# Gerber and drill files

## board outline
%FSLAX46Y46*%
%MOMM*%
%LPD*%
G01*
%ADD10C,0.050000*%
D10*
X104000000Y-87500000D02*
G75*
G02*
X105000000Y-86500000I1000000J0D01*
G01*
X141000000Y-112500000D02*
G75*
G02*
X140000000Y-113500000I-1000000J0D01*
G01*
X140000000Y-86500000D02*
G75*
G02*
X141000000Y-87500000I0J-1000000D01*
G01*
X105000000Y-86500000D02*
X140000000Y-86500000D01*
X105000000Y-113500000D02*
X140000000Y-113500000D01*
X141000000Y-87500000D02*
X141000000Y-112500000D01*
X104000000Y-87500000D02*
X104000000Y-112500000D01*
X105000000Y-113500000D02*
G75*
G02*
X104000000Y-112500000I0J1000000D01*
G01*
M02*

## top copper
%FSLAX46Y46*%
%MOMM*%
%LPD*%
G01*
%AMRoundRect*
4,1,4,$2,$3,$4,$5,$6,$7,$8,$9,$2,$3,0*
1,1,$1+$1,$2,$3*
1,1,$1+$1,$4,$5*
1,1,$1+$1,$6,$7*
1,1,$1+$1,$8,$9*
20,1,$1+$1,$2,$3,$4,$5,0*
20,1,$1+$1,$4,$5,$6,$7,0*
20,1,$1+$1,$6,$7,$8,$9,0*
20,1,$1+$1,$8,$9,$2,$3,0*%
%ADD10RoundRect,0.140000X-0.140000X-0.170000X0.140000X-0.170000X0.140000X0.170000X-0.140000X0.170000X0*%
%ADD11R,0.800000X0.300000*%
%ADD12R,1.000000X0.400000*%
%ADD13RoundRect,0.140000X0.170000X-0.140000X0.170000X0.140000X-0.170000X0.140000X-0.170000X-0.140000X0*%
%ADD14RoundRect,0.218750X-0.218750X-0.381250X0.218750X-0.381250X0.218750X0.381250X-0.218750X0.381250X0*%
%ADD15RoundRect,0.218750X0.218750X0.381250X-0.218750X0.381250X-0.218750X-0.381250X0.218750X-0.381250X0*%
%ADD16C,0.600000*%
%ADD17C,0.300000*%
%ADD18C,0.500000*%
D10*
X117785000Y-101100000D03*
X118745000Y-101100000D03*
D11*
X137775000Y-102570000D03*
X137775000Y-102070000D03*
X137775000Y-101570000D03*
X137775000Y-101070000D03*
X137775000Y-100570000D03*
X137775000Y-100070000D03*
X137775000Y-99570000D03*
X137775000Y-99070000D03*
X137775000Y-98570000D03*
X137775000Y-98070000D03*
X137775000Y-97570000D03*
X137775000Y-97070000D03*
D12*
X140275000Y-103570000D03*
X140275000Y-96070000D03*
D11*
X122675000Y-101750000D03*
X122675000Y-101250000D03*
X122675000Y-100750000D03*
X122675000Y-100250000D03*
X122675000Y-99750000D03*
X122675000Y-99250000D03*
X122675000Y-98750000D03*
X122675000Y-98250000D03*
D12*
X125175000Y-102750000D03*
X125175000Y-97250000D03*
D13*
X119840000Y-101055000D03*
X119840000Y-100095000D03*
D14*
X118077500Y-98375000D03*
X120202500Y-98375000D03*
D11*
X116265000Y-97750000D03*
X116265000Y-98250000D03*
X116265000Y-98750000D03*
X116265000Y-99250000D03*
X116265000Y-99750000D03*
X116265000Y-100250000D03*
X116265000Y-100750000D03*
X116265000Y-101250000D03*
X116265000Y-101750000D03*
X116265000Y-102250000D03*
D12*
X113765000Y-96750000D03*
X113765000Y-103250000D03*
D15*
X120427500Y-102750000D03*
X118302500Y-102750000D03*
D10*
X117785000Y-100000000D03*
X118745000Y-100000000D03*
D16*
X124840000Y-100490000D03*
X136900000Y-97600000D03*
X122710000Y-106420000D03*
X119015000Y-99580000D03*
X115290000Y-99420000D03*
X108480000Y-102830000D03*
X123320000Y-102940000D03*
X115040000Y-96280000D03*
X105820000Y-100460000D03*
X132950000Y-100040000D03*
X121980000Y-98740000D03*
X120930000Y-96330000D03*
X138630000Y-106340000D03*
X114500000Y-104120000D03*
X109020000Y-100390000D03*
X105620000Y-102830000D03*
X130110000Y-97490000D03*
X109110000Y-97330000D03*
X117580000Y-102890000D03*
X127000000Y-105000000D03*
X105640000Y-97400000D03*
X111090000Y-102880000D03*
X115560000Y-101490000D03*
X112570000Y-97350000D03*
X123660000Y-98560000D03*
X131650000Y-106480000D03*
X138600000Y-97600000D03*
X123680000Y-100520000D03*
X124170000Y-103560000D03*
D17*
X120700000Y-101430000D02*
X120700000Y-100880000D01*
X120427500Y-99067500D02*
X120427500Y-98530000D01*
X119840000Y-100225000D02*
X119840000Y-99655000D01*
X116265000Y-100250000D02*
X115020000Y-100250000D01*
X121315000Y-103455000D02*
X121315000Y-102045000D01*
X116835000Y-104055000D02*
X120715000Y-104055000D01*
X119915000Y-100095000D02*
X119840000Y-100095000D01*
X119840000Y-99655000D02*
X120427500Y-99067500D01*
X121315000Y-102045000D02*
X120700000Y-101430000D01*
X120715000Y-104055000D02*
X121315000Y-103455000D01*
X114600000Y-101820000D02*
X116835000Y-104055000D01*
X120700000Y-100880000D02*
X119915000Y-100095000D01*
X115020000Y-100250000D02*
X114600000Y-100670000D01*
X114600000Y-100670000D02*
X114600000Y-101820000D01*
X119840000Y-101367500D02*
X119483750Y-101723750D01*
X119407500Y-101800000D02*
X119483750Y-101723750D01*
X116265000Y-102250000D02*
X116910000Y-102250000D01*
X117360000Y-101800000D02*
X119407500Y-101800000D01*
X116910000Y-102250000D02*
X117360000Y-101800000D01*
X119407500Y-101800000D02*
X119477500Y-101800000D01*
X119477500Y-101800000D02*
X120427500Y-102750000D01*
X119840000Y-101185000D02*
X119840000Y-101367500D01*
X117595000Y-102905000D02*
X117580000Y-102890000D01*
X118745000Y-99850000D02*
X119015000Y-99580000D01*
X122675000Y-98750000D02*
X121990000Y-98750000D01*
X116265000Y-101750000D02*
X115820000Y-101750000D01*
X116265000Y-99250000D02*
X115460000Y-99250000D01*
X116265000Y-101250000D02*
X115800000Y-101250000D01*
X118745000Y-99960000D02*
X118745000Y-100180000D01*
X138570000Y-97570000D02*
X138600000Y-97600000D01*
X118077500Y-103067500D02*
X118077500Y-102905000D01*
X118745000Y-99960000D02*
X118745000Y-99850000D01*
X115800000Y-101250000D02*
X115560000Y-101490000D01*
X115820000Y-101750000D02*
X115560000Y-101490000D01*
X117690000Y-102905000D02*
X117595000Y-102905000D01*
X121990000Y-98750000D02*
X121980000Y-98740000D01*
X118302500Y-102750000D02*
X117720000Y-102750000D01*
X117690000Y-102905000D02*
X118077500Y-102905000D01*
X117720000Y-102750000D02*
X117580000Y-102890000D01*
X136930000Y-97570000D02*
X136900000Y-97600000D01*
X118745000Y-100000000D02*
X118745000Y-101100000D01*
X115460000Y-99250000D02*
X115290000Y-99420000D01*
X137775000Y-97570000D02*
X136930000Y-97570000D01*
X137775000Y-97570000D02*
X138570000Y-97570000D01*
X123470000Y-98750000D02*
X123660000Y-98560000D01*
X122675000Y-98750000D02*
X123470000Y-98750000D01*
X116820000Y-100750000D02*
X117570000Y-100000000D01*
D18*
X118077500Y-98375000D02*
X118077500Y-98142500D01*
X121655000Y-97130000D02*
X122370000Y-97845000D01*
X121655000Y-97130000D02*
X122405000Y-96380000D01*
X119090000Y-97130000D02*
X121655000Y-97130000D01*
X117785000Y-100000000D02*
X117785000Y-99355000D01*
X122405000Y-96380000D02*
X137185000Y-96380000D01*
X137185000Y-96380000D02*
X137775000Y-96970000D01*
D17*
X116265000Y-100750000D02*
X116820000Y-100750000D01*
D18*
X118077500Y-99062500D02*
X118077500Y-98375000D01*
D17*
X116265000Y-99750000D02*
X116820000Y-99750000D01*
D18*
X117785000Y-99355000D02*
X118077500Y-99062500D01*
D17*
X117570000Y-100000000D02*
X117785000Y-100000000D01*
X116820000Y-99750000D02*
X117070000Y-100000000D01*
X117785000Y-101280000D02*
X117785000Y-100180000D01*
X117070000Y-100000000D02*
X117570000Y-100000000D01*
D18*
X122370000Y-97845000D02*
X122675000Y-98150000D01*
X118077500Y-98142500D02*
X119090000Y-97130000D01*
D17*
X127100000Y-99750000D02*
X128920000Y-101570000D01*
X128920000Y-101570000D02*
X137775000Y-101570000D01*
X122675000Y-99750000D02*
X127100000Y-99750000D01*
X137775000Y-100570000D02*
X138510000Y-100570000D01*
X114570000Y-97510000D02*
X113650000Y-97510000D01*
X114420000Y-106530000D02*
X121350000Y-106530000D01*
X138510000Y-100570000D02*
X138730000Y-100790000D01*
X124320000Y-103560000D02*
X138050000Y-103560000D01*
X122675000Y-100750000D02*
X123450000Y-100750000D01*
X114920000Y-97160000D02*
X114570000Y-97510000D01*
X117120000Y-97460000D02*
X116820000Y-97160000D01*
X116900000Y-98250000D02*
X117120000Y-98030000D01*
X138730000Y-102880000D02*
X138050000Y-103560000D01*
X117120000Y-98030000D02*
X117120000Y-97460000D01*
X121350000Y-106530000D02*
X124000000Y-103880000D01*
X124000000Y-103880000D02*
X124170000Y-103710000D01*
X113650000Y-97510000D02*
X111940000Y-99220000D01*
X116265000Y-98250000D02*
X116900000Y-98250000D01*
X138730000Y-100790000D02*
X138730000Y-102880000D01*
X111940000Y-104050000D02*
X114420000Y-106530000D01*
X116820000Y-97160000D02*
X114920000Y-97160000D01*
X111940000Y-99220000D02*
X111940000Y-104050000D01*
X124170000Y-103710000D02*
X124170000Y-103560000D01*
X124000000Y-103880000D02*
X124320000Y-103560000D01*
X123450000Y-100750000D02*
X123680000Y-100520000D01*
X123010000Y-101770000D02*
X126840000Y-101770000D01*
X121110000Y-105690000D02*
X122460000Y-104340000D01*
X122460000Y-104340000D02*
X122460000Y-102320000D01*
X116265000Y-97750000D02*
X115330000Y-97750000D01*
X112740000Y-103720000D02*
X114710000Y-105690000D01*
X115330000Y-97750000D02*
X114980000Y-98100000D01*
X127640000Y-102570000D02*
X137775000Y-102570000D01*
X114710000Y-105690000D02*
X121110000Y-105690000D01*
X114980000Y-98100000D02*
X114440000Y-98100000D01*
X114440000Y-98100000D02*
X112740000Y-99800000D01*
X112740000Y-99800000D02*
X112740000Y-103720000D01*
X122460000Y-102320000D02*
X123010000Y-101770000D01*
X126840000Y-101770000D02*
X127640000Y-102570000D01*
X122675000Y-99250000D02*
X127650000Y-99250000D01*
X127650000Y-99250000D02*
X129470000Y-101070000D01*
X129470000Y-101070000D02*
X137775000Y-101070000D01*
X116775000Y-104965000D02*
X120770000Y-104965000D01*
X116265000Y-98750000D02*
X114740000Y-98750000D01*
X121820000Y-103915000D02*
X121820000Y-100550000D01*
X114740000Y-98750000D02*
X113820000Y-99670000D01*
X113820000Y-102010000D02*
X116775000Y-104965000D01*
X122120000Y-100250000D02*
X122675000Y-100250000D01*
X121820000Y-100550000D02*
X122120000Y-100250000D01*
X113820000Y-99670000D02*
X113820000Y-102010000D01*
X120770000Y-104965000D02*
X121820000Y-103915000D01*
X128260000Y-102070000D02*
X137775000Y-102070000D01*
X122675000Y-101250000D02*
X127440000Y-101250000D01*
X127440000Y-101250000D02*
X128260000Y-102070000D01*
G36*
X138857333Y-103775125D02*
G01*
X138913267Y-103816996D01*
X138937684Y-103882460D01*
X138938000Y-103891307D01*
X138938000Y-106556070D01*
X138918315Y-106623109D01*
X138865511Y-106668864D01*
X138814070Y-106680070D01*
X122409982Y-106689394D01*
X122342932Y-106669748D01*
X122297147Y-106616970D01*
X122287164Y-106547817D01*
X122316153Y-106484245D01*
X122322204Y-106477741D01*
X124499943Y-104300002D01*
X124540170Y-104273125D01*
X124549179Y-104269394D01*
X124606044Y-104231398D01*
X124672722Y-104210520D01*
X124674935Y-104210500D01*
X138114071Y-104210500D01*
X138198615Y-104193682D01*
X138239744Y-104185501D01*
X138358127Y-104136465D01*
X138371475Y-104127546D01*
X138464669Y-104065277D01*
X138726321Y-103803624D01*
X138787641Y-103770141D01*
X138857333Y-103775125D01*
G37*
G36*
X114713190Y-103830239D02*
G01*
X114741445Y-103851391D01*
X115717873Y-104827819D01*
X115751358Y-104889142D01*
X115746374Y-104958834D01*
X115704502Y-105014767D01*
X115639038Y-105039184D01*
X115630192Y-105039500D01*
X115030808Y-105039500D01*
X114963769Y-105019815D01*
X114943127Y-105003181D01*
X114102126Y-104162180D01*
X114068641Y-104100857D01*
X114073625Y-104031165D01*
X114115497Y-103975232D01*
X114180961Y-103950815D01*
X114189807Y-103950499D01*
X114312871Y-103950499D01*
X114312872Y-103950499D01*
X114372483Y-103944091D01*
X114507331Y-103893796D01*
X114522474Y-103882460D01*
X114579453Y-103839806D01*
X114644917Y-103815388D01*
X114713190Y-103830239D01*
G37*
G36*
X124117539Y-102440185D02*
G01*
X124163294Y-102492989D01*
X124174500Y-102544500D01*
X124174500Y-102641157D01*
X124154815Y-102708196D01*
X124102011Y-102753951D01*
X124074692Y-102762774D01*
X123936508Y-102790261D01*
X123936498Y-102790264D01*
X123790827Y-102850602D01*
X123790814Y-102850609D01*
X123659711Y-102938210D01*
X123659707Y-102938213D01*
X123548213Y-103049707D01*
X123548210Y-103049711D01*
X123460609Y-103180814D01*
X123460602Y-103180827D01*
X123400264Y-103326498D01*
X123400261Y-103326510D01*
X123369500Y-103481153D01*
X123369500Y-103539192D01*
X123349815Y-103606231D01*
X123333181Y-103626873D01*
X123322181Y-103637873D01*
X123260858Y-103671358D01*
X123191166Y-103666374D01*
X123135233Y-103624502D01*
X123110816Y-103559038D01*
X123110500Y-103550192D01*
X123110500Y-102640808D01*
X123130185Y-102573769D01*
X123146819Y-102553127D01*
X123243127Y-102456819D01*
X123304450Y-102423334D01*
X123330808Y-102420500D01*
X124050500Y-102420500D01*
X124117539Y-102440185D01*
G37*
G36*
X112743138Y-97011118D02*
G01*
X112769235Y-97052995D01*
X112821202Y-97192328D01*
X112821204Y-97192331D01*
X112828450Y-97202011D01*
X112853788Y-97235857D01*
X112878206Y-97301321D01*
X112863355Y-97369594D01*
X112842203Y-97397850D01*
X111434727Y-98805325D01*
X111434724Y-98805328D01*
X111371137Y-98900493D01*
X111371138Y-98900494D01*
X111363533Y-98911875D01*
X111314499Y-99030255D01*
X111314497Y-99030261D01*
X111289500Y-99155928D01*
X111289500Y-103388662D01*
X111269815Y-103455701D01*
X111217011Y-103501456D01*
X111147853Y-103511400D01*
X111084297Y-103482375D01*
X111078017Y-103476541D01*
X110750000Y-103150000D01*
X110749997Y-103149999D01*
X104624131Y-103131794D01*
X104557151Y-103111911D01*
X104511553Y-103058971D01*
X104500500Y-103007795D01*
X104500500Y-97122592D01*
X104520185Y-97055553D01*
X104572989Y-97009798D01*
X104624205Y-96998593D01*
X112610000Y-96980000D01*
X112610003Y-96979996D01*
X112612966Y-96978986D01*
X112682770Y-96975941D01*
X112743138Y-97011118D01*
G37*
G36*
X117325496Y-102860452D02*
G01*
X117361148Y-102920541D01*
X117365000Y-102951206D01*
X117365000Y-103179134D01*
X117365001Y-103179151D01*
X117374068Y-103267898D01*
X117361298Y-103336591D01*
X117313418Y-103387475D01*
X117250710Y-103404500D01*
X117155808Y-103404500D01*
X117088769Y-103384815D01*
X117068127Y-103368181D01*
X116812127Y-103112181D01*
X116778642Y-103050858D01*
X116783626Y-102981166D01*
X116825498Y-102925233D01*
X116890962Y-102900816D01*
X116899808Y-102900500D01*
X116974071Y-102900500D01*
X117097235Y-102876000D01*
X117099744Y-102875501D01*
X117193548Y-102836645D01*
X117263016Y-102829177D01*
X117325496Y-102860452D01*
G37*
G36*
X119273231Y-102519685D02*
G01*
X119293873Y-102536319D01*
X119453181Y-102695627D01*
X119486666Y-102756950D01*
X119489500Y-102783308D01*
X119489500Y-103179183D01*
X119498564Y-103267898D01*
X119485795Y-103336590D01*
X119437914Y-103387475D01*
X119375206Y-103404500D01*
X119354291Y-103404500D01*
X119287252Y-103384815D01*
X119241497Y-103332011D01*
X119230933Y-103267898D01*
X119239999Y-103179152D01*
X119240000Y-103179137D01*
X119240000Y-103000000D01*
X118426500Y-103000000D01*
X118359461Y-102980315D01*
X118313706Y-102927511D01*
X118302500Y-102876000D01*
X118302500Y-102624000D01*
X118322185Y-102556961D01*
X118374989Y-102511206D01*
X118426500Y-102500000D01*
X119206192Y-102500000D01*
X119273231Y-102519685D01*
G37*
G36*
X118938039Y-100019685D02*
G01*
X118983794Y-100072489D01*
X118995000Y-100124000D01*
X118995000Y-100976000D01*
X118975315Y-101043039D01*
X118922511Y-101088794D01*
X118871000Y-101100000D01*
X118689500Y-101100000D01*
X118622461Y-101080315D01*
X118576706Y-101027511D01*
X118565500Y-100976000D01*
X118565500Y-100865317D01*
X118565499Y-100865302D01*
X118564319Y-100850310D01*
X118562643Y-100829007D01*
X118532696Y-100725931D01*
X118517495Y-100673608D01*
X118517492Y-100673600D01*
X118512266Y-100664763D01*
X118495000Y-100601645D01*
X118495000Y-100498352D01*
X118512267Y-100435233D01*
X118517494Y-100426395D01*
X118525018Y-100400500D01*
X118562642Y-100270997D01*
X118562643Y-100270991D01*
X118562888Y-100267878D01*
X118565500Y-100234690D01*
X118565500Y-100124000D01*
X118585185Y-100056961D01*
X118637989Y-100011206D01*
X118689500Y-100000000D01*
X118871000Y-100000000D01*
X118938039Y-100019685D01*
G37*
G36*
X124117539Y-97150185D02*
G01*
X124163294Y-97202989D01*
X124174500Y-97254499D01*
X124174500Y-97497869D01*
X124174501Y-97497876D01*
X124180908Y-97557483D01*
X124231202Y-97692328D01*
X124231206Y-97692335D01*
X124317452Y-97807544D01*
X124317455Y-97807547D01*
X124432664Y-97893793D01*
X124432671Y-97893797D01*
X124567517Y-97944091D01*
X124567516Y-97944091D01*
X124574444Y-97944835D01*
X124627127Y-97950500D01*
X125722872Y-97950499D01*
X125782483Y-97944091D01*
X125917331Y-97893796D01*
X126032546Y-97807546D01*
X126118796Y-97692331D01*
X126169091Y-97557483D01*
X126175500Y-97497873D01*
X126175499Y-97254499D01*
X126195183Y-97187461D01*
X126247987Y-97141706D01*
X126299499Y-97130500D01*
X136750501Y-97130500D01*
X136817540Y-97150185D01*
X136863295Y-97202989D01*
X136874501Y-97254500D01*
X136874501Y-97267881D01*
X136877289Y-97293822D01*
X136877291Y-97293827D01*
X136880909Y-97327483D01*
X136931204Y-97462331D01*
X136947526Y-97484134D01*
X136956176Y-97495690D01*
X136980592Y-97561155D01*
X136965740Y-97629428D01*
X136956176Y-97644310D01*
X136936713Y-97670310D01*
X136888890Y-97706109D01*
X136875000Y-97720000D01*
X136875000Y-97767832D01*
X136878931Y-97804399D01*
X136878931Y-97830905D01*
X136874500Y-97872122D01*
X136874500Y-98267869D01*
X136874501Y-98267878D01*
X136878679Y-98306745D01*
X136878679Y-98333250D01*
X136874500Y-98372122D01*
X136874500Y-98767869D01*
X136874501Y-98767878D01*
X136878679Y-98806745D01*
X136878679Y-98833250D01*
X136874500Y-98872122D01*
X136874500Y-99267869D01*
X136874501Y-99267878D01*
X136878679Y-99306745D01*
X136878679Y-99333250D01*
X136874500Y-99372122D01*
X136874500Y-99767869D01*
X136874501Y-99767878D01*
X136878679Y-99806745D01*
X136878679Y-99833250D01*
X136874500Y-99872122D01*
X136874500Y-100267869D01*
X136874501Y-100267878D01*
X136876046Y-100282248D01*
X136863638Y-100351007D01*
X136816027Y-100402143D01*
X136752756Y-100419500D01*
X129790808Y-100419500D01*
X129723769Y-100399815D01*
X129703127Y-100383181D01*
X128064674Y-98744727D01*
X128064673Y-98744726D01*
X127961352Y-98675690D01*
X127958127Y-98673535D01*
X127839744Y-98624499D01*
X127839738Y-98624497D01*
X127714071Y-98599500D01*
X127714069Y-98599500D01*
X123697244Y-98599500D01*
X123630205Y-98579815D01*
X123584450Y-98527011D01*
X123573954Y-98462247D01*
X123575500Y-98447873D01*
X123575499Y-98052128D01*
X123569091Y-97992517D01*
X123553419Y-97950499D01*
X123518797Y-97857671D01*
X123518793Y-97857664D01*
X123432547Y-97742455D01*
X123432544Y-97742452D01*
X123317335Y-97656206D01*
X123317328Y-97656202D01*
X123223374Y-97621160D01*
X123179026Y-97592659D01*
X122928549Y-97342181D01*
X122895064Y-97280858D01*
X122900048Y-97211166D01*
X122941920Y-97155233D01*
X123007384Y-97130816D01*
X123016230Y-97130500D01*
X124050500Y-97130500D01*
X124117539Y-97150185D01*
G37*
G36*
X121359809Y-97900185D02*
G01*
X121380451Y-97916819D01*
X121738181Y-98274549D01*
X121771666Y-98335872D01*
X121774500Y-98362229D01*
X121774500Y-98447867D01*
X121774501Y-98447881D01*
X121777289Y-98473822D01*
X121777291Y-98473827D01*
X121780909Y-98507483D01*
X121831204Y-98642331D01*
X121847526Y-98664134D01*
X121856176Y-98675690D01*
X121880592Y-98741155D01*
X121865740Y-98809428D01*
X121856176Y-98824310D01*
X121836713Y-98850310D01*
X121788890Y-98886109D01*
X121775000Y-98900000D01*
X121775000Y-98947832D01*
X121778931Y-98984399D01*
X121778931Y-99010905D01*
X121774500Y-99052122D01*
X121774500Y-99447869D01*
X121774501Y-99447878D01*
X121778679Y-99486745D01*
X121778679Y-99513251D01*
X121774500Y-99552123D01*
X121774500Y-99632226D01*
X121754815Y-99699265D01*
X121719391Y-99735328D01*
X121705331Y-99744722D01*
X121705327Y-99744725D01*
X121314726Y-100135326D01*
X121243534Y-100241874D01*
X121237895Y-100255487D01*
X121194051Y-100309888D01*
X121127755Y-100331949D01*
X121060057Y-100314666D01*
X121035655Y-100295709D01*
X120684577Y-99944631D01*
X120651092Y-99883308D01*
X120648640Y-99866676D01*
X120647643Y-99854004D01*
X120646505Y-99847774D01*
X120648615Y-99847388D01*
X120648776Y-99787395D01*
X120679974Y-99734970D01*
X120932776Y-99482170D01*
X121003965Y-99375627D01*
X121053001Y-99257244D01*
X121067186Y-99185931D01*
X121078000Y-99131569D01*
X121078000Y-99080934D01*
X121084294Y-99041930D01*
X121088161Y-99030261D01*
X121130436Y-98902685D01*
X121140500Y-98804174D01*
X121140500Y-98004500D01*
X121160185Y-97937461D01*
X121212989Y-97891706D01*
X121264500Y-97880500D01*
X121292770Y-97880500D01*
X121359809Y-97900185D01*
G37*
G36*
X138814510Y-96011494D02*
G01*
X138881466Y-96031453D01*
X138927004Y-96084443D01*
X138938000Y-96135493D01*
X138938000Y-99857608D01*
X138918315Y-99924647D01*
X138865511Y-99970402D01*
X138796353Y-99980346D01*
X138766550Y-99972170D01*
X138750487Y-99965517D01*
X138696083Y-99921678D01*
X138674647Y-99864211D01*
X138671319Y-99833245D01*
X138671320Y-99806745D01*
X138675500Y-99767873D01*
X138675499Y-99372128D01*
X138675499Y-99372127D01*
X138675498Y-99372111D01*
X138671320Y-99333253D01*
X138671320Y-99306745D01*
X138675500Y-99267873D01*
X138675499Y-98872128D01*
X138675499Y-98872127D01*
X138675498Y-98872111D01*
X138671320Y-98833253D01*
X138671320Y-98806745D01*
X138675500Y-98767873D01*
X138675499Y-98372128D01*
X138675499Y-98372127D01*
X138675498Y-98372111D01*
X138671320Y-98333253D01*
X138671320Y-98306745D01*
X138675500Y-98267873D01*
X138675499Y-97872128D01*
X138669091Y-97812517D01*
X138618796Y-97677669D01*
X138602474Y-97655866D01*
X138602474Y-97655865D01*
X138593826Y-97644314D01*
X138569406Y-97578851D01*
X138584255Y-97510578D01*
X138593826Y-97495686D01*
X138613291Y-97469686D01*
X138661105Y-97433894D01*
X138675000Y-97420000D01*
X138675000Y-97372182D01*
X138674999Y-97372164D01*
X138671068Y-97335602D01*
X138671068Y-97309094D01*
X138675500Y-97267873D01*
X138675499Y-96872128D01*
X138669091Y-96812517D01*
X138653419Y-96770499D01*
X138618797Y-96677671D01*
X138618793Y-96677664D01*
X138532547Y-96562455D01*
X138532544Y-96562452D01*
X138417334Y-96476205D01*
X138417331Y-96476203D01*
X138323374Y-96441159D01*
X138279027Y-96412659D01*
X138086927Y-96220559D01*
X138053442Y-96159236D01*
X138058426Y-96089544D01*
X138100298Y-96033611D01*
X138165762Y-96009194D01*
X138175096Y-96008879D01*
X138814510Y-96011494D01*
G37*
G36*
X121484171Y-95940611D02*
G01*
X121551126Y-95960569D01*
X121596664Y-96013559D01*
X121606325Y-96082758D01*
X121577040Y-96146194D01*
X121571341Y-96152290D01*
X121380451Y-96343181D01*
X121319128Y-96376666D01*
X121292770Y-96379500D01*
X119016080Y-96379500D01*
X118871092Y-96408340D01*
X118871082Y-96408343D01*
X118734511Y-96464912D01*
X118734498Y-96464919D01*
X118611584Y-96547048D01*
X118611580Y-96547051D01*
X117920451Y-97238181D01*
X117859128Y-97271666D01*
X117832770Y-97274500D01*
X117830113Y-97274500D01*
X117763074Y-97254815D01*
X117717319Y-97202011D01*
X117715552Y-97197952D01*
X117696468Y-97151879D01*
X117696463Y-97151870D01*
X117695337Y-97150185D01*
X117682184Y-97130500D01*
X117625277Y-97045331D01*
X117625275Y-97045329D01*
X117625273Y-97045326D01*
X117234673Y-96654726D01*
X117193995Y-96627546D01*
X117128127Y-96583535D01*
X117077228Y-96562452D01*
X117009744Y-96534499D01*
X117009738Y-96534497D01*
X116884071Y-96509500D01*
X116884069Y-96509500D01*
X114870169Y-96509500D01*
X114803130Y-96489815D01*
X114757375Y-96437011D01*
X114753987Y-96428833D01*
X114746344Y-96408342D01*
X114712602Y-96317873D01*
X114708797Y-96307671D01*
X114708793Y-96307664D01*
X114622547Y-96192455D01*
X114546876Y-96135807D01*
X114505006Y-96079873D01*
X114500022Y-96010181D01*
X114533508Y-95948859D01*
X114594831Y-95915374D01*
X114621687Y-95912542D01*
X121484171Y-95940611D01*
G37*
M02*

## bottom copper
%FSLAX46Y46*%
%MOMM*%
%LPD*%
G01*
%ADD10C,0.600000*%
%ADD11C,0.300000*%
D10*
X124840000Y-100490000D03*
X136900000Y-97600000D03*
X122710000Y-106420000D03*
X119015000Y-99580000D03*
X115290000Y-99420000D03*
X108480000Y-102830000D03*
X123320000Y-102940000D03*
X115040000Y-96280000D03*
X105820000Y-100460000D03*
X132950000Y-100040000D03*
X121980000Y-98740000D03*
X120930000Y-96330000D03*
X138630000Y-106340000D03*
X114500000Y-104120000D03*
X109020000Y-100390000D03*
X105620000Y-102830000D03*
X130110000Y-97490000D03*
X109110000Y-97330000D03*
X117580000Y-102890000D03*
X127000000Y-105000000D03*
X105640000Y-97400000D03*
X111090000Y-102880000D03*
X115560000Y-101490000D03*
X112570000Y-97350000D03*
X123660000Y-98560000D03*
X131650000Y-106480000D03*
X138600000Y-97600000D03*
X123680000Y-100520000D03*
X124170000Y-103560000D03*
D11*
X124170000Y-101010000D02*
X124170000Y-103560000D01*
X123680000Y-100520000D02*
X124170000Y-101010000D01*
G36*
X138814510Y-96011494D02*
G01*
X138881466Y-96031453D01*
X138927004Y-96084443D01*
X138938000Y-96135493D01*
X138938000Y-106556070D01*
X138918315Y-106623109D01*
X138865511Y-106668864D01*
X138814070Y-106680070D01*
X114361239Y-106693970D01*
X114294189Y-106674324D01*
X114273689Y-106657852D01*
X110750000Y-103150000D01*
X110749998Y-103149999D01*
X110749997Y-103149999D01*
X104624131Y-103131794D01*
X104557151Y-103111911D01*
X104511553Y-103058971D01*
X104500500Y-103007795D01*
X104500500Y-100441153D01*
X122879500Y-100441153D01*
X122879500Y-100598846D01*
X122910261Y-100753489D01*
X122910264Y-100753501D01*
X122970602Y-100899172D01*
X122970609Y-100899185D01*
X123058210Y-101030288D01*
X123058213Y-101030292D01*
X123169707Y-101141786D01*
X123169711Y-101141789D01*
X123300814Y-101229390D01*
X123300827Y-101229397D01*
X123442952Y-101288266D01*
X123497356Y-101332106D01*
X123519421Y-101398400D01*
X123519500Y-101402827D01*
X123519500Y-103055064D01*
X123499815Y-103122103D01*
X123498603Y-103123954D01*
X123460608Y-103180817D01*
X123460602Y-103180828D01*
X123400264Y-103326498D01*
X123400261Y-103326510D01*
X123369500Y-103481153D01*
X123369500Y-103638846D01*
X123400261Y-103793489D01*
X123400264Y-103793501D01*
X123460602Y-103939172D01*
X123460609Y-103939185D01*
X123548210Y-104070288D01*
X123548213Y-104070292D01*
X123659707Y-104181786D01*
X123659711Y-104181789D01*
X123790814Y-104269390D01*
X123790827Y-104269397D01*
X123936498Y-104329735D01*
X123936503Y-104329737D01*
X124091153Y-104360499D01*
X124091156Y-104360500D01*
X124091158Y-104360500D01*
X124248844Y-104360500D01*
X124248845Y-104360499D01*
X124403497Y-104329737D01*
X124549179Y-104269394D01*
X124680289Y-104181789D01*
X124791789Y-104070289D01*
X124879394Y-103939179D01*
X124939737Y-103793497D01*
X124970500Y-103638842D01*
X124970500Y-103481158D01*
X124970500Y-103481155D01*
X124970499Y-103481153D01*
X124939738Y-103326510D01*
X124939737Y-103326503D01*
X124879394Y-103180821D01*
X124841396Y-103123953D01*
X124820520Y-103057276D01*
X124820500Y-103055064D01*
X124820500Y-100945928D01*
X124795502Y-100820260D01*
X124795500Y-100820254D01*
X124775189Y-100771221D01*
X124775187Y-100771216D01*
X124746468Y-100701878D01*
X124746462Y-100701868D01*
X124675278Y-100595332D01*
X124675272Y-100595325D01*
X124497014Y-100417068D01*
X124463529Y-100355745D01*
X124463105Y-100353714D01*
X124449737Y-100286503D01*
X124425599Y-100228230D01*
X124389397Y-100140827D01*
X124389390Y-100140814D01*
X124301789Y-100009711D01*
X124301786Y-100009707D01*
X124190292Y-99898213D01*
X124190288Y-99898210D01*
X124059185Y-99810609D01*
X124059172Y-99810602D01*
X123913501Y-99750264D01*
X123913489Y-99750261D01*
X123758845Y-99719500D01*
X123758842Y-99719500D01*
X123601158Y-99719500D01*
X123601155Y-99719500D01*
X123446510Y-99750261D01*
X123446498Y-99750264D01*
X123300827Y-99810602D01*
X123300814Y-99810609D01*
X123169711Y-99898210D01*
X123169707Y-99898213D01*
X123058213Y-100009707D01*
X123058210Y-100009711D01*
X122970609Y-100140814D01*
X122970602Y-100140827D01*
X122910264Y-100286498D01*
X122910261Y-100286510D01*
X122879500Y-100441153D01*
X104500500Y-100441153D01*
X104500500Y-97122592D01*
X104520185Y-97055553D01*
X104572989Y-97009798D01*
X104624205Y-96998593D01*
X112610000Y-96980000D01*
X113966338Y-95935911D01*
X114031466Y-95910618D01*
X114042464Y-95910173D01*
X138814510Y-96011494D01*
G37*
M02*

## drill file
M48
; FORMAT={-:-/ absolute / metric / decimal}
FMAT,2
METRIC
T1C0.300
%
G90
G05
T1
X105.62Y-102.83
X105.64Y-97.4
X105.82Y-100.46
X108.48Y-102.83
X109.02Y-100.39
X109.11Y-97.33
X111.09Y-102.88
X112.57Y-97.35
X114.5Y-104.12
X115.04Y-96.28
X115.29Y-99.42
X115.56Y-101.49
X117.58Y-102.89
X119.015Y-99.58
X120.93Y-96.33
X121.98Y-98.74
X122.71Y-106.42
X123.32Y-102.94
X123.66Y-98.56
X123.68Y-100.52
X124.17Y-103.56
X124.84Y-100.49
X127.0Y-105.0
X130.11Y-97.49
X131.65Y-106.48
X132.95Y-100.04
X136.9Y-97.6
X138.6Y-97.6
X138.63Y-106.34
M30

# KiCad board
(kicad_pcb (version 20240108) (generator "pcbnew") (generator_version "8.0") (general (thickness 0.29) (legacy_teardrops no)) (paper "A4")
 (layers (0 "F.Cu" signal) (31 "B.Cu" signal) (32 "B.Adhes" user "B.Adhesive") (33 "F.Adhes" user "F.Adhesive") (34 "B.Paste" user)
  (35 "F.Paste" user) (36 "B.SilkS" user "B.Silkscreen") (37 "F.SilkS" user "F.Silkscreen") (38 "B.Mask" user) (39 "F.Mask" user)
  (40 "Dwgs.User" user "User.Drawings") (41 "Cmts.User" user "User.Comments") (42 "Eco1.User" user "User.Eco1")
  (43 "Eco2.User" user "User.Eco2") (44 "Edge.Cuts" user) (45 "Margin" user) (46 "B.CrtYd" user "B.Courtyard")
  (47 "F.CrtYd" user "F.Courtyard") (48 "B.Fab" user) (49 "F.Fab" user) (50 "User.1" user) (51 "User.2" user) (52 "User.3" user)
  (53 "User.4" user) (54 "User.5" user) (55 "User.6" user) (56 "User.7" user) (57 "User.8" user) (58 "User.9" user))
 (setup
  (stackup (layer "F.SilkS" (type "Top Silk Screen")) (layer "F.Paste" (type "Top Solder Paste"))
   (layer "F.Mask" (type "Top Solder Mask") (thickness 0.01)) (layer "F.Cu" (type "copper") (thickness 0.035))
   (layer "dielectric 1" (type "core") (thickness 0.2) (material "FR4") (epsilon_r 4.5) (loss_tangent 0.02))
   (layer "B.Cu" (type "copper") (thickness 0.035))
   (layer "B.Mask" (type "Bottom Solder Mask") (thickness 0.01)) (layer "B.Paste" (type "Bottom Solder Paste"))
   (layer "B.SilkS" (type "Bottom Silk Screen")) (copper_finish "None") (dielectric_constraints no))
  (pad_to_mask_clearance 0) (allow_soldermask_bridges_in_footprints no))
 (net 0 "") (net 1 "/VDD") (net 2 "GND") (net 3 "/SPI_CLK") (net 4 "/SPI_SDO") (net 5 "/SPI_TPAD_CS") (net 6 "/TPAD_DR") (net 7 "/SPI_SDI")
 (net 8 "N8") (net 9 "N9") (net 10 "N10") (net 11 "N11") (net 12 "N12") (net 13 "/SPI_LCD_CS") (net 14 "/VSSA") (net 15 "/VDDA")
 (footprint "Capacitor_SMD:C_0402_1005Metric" (layer "F.Cu") (at 118.265 101.1)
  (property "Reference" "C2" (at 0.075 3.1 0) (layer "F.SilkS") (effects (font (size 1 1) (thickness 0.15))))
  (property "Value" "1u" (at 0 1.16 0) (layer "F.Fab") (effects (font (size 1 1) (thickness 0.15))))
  (pad "1" smd roundrect (at -0.48 0) (size 0.56 0.62) (layers "F.Cu" "F.Paste" "F.Mask") (roundrect_rratio 0.25) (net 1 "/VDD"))
  (pad "2" smd roundrect (at 0.48 0) (size 0.56 0.62) (layers "F.Cu" "F.Paste" "F.Mask") (roundrect_rratio 0.25) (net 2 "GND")))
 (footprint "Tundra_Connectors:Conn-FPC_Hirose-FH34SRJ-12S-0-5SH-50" (layer "F.Cu") (at 138.8 99.82 90)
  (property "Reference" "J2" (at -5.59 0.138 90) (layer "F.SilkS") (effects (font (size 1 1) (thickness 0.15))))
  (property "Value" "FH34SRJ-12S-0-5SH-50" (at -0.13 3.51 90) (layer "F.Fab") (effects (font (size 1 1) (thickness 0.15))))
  (pad "1" smd rect (at -2.75 -1.025 90) (size 0.3 0.8) (layers "F.Cu" "F.Paste" "F.Mask") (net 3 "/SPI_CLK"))
  (pad "2" smd rect (at -2.25 -1.025 90) (size 0.3 0.8) (layers "F.Cu" "F.Paste" "F.Mask") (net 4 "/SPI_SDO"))
  (pad "3" smd rect (at -1.75 -1.025 90) (size 0.3 0.8) (layers "F.Cu" "F.Paste" "F.Mask") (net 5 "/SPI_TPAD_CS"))
  (pad "4" smd rect (at -1.25 -1.025 90) (size 0.3 0.8) (layers "F.Cu" "F.Paste" "F.Mask") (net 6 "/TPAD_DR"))
  (pad "5" smd rect (at -0.75 -1.025 90) (size 0.3 0.8) (layers "F.Cu" "F.Paste" "F.Mask") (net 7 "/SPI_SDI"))
  (pad "6" smd rect (at -0.25 -1.025 90) (size 0.3 0.8) (layers "F.Cu" "F.Paste" "F.Mask") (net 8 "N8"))
  (pad "7" smd rect (at 0.25 -1.025 90) (size 0.3 0.8) (layers "F.Cu" "F.Paste" "F.Mask") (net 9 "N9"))
  (pad "8" smd rect (at 0.75 -1.025 90) (size 0.3 0.8) (layers "F.Cu" "F.Paste" "F.Mask") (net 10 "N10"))
  (pad "9" smd rect (at 1.25 -1.025 90) (size 0.3 0.8) (layers "F.Cu" "F.Paste" "F.Mask") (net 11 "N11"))
  (pad "10" smd rect (at 1.75 -1.025 90) (size 0.3 0.8) (layers "F.Cu" "F.Paste" "F.Mask") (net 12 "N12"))
  (pad "11" smd rect (at 2.25 -1.025 90) (size 0.3 0.8) (layers "F.Cu" "F.Paste" "F.Mask") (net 2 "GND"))
  (pad "12" smd rect (at 2.75 -1.025 90) (size 0.3 0.8) (layers "F.Cu" "F.Paste" "F.Mask") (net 1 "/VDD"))
  (pad "MP" smd rect (at -3.75 1.475 90) (size 0.4 1) (layers "F.Cu" "F.Paste" "F.Mask"))
  (pad "MP" smd rect (at 3.75 1.475 90) (size 0.4 1) (layers "F.Cu" "F.Paste" "F.Mask")))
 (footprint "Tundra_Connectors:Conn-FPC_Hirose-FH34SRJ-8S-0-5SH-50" (layer "F.Cu") (at 123.7 100 90)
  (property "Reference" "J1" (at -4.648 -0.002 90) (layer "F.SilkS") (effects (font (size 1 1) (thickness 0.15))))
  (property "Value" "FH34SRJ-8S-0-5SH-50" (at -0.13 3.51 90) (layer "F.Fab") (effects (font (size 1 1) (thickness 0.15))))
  (pad "1" smd rect (at -1.75 -1.025 90) (size 0.3 0.8) (layers "F.Cu" "F.Paste" "F.Mask") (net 3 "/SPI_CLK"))
  (pad "2" smd rect (at -1.25 -1.025 90) (size 0.3 0.8) (layers "F.Cu" "F.Paste" "F.Mask") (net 4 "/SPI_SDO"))
  (pad "3" smd rect (at -0.75 -1.025 90) (size 0.3 0.8) (layers "F.Cu" "F.Paste" "F.Mask") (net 7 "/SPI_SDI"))
  (pad "4" smd rect (at -0.25 -1.025 90) (size 0.3 0.8) (layers "F.Cu" "F.Paste" "F.Mask") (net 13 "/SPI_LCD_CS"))
  (pad "5" smd rect (at 0.25 -1.025 90) (size 0.3 0.8) (layers "F.Cu" "F.Paste" "F.Mask") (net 5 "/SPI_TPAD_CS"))
  (pad "6" smd rect (at 0.75 -1.025 90) (size 0.3 0.8) (layers "F.Cu" "F.Paste" "F.Mask") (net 6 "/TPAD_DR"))
  (pad "7" smd rect (at 1.25 -1.025 90) (size 0.3 0.8) (layers "F.Cu" "F.Paste" "F.Mask") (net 2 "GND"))
  (pad "8" smd rect (at 1.75 -1.025 90) (size 0.3 0.8) (layers "F.Cu" "F.Paste" "F.Mask") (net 1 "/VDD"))
  (pad "MP" smd rect (at -2.75 1.475 90) (size 0.4 1) (layers "F.Cu" "F.Paste" "F.Mask"))
  (pad "MP" smd rect (at 2.75 1.475 90) (size 0.4 1) (layers "F.Cu" "F.Paste" "F.Mask")))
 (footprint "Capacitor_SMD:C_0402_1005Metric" (layer "F.Cu") (at 119.84 100.575 90)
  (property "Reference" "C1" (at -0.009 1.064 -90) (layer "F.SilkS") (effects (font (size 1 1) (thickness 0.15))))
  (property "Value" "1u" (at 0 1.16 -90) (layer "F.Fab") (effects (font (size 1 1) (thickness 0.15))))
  (pad "1" smd roundrect (at -0.48 0 90) (size 0.56 0.62) (layers "F.Cu" "F.Paste" "F.Mask") (roundrect_rratio 0.25) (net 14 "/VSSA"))
  (pad "2" smd roundrect (at 0.48 0 90) (size 0.56 0.62) (layers "F.Cu" "F.Paste" "F.Mask") (roundrect_rratio 0.25) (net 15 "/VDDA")))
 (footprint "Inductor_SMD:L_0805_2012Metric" (layer "F.Cu") (at 119.14 98.375)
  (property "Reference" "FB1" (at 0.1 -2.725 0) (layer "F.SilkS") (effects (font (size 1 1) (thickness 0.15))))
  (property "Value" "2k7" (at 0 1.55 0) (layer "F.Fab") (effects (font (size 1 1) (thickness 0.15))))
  (pad "1" smd roundrect (at -1.0625 0) (size 0.875 1.2) (layers "F.Cu" "F.Paste" "F.Mask") (roundrect_rratio 0.25) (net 1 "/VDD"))
  (pad "2" smd roundrect (at 1.0625 0) (size 0.875 1.2) (layers "F.Cu" "F.Paste" "F.Mask") (roundrect_rratio 0.25) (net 15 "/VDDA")))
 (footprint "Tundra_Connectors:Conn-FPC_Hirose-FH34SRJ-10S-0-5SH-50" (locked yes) (layer "F.Cu") (at 115.24 100 -90)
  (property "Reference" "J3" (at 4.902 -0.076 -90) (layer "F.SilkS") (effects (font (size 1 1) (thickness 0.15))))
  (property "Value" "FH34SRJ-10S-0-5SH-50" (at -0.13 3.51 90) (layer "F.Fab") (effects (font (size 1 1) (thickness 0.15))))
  (pad "1" smd rect (at -2.25 -1.025 270) (size 0.3 0.8) (layers "F.Cu" "F.Paste" "F.Mask") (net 3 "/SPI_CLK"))
  (pad "2" smd rect (at -1.75 -1.025 270) (size 0.3 0.8) (layers "F.Cu" "F.Paste" "F.Mask") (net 7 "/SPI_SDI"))
  (pad "3" smd rect (at -1.25 -1.025 270) (size 0.3 0.8) (layers "F.Cu" "F.Paste" "F.Mask") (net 13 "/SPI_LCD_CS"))
  (pad "4" smd rect (at -0.75 -1.025 270) (size 0.3 0.8) (layers "F.Cu" "F.Paste" "F.Mask") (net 2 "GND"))
  (pad "5" smd rect (at -0.25 -1.025 270) (size 0.3 0.8) (layers "F.Cu" "F.Paste" "F.Mask") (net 1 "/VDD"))
  (pad "6" smd rect (at 0.25 -1.025 270) (size 0.3 0.8) (layers "F.Cu" "F.Paste" "F.Mask") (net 15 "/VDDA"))
  (pad "7" smd rect (at 0.75 -1.025 270) (size 0.3 0.8) (layers "F.Cu" "F.Paste" "F.Mask") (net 1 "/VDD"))
  (pad "8" smd rect (at 1.25 -1.025 270) (size 0.3 0.8) (layers "F.Cu" "F.Paste" "F.Mask") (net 2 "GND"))
  (pad "9" smd rect (at 1.75 -1.025 270) (size 0.3 0.8) (layers "F.Cu" "F.Paste" "F.Mask") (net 2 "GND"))
  (pad "10" smd rect (at 2.25 -1.025 270) (size 0.3 0.8) (layers "F.Cu" "F.Paste" "F.Mask") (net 14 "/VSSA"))
  (pad "MP" smd rect (at -3.25 1.475 270) (size 0.4 1) (layers "F.Cu" "F.Paste" "F.Mask"))
  (pad "MP" smd rect (at 3.25 1.475 270) (size 0.4 1) (layers "F.Cu" "F.Paste" "F.Mask")))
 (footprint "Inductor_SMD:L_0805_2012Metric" (layer "F.Cu") (at 119.365 102.75 180)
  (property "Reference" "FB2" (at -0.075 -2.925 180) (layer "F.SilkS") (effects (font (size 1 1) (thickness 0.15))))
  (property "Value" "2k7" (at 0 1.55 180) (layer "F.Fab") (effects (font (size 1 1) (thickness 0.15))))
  (pad "1" smd roundrect (at -1.0625 0 180) (size 0.875 1.2) (layers "F.Cu" "F.Paste" "F.Mask") (roundrect_rratio 0.25) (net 14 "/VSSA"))
  (pad "2" smd roundrect (at 1.0625 0 180) (size 0.875 1.2) (layers "F.Cu" "F.Paste" "F.Mask") (roundrect_rratio 0.25) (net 2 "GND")))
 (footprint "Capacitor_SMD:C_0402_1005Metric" (layer "F.Cu") (at 118.265 100)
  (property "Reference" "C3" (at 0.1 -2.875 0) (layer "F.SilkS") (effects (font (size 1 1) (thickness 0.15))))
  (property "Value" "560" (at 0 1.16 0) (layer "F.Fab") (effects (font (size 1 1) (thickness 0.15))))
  (pad "1" smd roundrect (at -0.48 0) (size 0.56 0.62) (layers "F.Cu" "F.Paste" "F.Mask") (roundrect_rratio 0.25) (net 1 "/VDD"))
  (pad "2" smd roundrect (at 0.48 0) (size 0.56 0.62) (layers "F.Cu" "F.Paste" "F.Mask") (roundrect_rratio 0.25) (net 2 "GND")))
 (gr_arc (start 104 87.5) (mid 104.292893 86.792893) (end 105 86.5) (stroke (width 0.05) (type default)) (layer "Edge.Cuts"))
 (gr_arc (start 141 112.5) (mid 140.707107 113.207107) (end 140 113.5) (stroke (width 0.05) (type default)) (layer "Edge.Cuts"))
 (gr_arc (start 140 86.5) (mid 140.707107 86.792893) (end 141 87.5) (stroke (width 0.05) (type default)) (layer "Edge.Cuts"))
 (gr_line (start 105 86.5) (end 140 86.5) (stroke (width 0.05) (type default)) (layer "Edge.Cuts"))
 (gr_line (start 105 113.5) (end 140 113.5) (stroke (width 0.05) (type default)) (layer "Edge.Cuts"))
 (gr_line (start 141 87.5) (end 141 112.5) (stroke (width 0.05) (type default)) (layer "Edge.Cuts"))
 (gr_line (start 104 87.5) (end 104 112.5) (stroke (width 0.05) (type default)) (layer "Edge.Cuts"))
 (gr_arc (start 105 113.5) (mid 104.292893 113.207107) (end 104 112.5) (stroke (width 0.05) (type default)) (layer "Edge.Cuts"))
 (segment (start 120.7 101.43) (end 120.7 100.88) (width 0.3) (layer "F.Cu") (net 15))
 (segment (start 120.4275 99.0675) (end 120.4275 98.53) (width 0.3) (layer "F.Cu") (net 15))
 (segment (start 119.84 100.225) (end 119.84 99.655) (width 0.3) (layer "F.Cu") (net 15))
 (segment (start 116.265 100.25) (end 115.02 100.25) (width 0.3) (layer "F.Cu") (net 15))
 (segment (start 121.315 103.455) (end 121.315 102.045) (width 0.3) (layer "F.Cu") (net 15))
 (segment (start 116.835 104.055) (end 120.715 104.055) (width 0.3) (layer "F.Cu") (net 15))
 (segment (start 119.915 100.095) (end 119.84 100.095) (width 0.3) (layer "F.Cu") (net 15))
 (segment (start 119.84 99.655) (end 120.4275 99.0675) (width 0.3) (layer "F.Cu") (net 15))
 (segment (start 121.315 102.045) (end 120.7 101.43) (width 0.3) (layer "F.Cu") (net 15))
 (segment (start 120.715 104.055) (end 121.315 103.455) (width 0.3) (layer "F.Cu") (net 15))
 (segment (start 114.6 101.82) (end 116.835 104.055) (width 0.3) (layer "F.Cu") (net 15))
 (segment (start 120.7 100.88) (end 119.915 100.095) (width 0.3) (layer "F.Cu") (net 15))
 (segment (start 115.02 100.25) (end 114.6 100.67) (width 0.3) (layer "F.Cu") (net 15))
 (segment (start 114.6 100.67) (end 114.6 101.82) (width 0.3) (layer "F.Cu") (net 15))
 (segment (start 119.84 101.3675) (end 119.48375 101.72375) (width 0.3) (layer "F.Cu") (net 14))
 (segment (start 119.4075 101.8) (end 119.48375 101.72375) (width 0.3) (layer "F.Cu") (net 14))
 (segment (start 116.265 102.25) (end 116.91 102.25) (width 0.3) (layer "F.Cu") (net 14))
 (segment (start 117.36 101.8) (end 119.4075 101.8) (width 0.3) (layer "F.Cu") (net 14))
 (segment (start 116.91 102.25) (end 117.36 101.8) (width 0.3) (layer "F.Cu") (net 14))
 (segment (start 119.4075 101.8) (end 119.4775 101.8) (width 0.3) (layer "F.Cu") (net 14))
 (segment (start 119.4775 101.8) (end 120.4275 102.75) (width 0.3) (layer "F.Cu") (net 14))
 (segment (start 119.84 101.185) (end 119.84 101.3675) (width 0.3) (layer "F.Cu") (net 14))
 (segment (start 117.595 102.905) (end 117.58 102.89) (width 0.3) (layer "F.Cu") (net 2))
 (segment (start 118.745 99.85) (end 119.015 99.58) (width 0.3) (layer "F.Cu") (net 2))
 (segment (start 122.675 98.75) (end 121.99 98.75) (width 0.3) (layer "F.Cu") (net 2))
 (segment (start 116.265 101.75) (end 115.82 101.75) (width 0.3) (layer "F.Cu") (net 2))
 (segment (start 116.265 99.25) (end 115.46 99.25) (width 0.3) (layer "F.Cu") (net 2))
 (segment (start 116.265 101.25) (end 115.8 101.25) (width 0.3) (layer "F.Cu") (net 2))
 (segment (start 118.745 99.96) (end 118.745 100.18) (width 0.3) (layer "F.Cu") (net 2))
 (segment (start 138.57 97.57) (end 138.6 97.6) (width 0.3) (layer "F.Cu") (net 2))
 (segment (start 118.0775 103.0675) (end 118.0775 102.905) (width 0.3) (layer "F.Cu") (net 2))
 (segment (start 118.745 99.96) (end 118.745 99.85) (width 0.3) (layer "F.Cu") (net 2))
 (segment (start 115.8 101.25) (end 115.56 101.49) (width 0.3) (layer "F.Cu") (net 2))
 (segment (start 115.82 101.75) (end 115.56 101.49) (width 0.3) (layer "F.Cu") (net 2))
 (segment (start 117.69 102.905) (end 117.595 102.905) (width 0.3) (layer "F.Cu") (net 2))
 (segment (start 121.99 98.75) (end 121.98 98.74) (width 0.3) (layer "F.Cu") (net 2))
 (segment (start 118.3025 102.75) (end 117.72 102.75) (width 0.3) (layer "F.Cu") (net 2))
 (segment (start 117.69 102.905) (end 118.0775 102.905) (width 0.3) (layer "F.Cu") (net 2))
 (segment (start 117.72 102.75) (end 117.58 102.89) (width 0.3) (layer "F.Cu") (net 2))
 (segment (start 136.93 97.57) (end 136.9 97.6) (width 0.3) (layer "F.Cu") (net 2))
 (segment (start 118.745 100) (end 118.745 101.1) (width 0.3) (layer "F.Cu") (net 2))
 (segment (start 115.46 99.25) (end 115.29 99.42) (width 0.3) (layer "F.Cu") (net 2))
 (segment (start 137.775 97.57) (end 136.93 97.57) (width 0.3) (layer "F.Cu") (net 2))
 (segment (start 137.775 97.57) (end 138.57 97.57) (width 0.3) (layer "F.Cu") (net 2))
 (segment (start 123.47 98.75) (end 123.66 98.56) (width 0.3) (layer "F.Cu") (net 2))
 (segment (start 122.675 98.75) (end 123.47 98.75) (width 0.3) (layer "F.Cu") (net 2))
 (via (at 124.84 100.49) (size 0.6) (drill 0.3) (layers "F.Cu" "B.Cu") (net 2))
 (via (at 136.9 97.6) (size 0.6) (drill 0.3) (layers "F.Cu" "B.Cu") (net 2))
 (via (at 122.71 106.42) (size 0.6) (drill 0.3) (layers "F.Cu" "B.Cu") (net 2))
 (via (at 119.015 99.58) (size 0.6) (drill 0.3) (layers "F.Cu" "B.Cu") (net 2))
 (via (at 115.29 99.42) (size 0.6) (drill 0.3) (layers "F.Cu" "B.Cu") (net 2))
 (via (at 108.48 102.83) (size 0.6) (drill 0.3) (layers "F.Cu" "B.Cu") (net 2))
 (via (at 123.32 102.94) (size 0.6) (drill 0.3) (layers "F.Cu" "B.Cu") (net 2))
 (via (at 115.04 96.28) (size 0.6) (drill 0.3) (layers "F.Cu" "B.Cu") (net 2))
 (via (at 105.82 100.46) (size 0.6) (drill 0.3) (layers "F.Cu" "B.Cu") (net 2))
 (via (at 132.95 100.04) (size 0.6) (drill 0.3) (layers "F.Cu" "B.Cu") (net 2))
 (via (at 121.98 98.74) (size 0.6) (drill 0.3) (layers "F.Cu" "B.Cu") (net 2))
 (via (at 120.93 96.33) (size 0.6) (drill 0.3) (layers "F.Cu" "B.Cu") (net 2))
 (via (at 138.63 106.34) (size 0.6) (drill 0.3) (layers "F.Cu" "B.Cu") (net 2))
 (via (at 114.5 104.12) (size 0.6) (drill 0.3) (layers "F.Cu" "B.Cu") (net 2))
 (via (at 109.02 100.39) (size 0.6) (drill 0.3) (layers "F.Cu" "B.Cu") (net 2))
 (via (at 105.62 102.83) (size 0.6) (drill 0.3) (layers "F.Cu" "B.Cu") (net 2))
 (via (at 130.11 97.49) (size 0.6) (drill 0.3) (layers "F.Cu" "B.Cu") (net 2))
 (via (at 109.11 97.33) (size 0.6) (drill 0.3) (layers "F.Cu" "B.Cu") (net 2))
 (via (at 117.58 102.89) (size 0.6) (drill 0.3) (layers "F.Cu" "B.Cu") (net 2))
 (via (at 127 105) (size 0.6) (drill 0.3) (layers "F.Cu" "B.Cu") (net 2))
 (via (at 105.64 97.4) (size 0.6) (drill 0.3) (layers "F.Cu" "B.Cu") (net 2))
 (via (at 111.09 102.88) (size 0.6) (drill 0.3) (layers "F.Cu" "B.Cu") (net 2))
 (via (at 115.56 101.49) (size 0.6) (drill 0.3) (layers "F.Cu" "B.Cu") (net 2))
 (via (at 112.57 97.35) (size 0.6) (drill 0.3) (layers "F.Cu" "B.Cu") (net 2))
 (via (at 123.66 98.56) (size 0.6) (drill 0.3) (layers "F.Cu" "B.Cu") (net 2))
 (via (at 131.65 106.48) (size 0.6) (drill 0.3) (layers "F.Cu" "B.Cu") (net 2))
 (via (at 138.6 97.6) (size 0.6) (drill 0.3) (layers "F.Cu" "B.Cu") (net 2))
 (segment (start 116.82 100.75) (end 117.57 100) (width 0.3) (layer "F.Cu") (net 1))
 (segment (start 118.0775 98.375) (end 118.0775 98.1425) (width 0.5) (layer "F.Cu") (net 1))
 (segment (start 121.655 97.13) (end 122.37 97.845) (width 0.5) (layer "F.Cu") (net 1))
 (segment (start 121.655 97.13) (end 122.405 96.38) (width 0.5) (layer "F.Cu") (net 1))
 (segment (start 119.09 97.13) (end 121.655 97.13) (width 0.5) (layer "F.Cu") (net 1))
 (segment (start 117.785 100) (end 117.785 99.355) (width 0.5) (layer "F.Cu") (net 1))
 (segment (start 122.405 96.38) (end 137.185 96.38) (width 0.5) (layer "F.Cu") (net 1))
 (segment (start 137.185 96.38) (end 137.775 96.97) (width 0.5) (layer "F.Cu") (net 1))
 (segment (start 116.265 100.75) (end 116.82 100.75) (width 0.3) (layer "F.Cu") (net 1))
 (segment (start 118.0775 99.0625) (end 118.0775 98.375) (width 0.5) (layer "F.Cu") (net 1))
 (segment (start 116.265 99.75) (end 116.82 99.75) (width 0.3) (layer "F.Cu") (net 1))
 (segment (start 117.785 99.355) (end 118.0775 99.0625) (width 0.5) (layer "F.Cu") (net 1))
 (segment (start 117.57 100) (end 117.785 100) (width 0.3) (layer "F.Cu") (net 1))
 (segment (start 116.82 99.75) (end 117.07 100) (width 0.3) (layer "F.Cu") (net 1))
 (segment (start 117.785 101.28) (end 117.785 100.18) (width 0.3) (layer "F.Cu") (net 1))
 (segment (start 117.07 100) (end 117.57 100) (width 0.3) (layer "F.Cu") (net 1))
 (segment (start 122.37 97.845) (end 122.675 98.15) (width 0.5) (layer "F.Cu") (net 1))
 (segment (start 118.0775 98.1425) (end 119.09 97.13) (width 0.5) (layer "F.Cu") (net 1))
 (segment (start 127.1 99.75) (end 128.92 101.57) (width 0.3) (layer "F.Cu") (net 5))
 (segment (start 128.92 101.57) (end 137.775 101.57) (width 0.3) (layer "F.Cu") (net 5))
 (segment (start 122.675 99.75) (end 127.1 99.75) (width 0.3) (layer "F.Cu") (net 5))
 (segment (start 137.775 100.57) (end 138.51 100.57) (width 0.3) (layer "F.Cu") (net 7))
 (segment (start 114.57 97.51) (end 113.65 97.51) (width 0.3) (layer "F.Cu") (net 7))
 (segment (start 114.42 106.53) (end 121.35 106.53) (width 0.3) (layer "F.Cu") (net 7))
 (segment (start 138.51 100.57) (end 138.73 100.79) (width 0.3) (layer "F.Cu") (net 7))
 (segment (start 124.32 103.56) (end 138.05 103.56) (width 0.3) (layer "F.Cu") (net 7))
 (segment (start 122.675 100.75) (end 123.45 100.75) (width 0.3) (layer "F.Cu") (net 7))
 (segment (start 114.92 97.16) (end 114.57 97.51) (width 0.3) (layer "F.Cu") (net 7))
 (segment (start 117.12 97.46) (end 116.82 97.16) (width 0.3) (layer "F.Cu") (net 7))
 (segment (start 116.9 98.25) (end 117.12 98.03) (width 0.3) (layer "F.Cu") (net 7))
 (segment (start 138.73 102.88) (end 138.05 103.56) (width 0.3) (layer "F.Cu") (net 7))
 (segment (start 117.12 98.03) (end 117.12 97.46) (width 0.3) (layer "F.Cu") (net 7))
 (segment (start 121.35 106.53) (end 124 103.88) (width 0.3) (layer "F.Cu") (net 7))
 (segment (start 124 103.88) (end 124.17 103.71) (width 0.3) (layer "F.Cu") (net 7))
 (segment (start 113.65 97.51) (end 111.94 99.22) (width 0.3) (layer "F.Cu") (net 7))
 (segment (start 116.265 98.25) (end 116.9 98.25) (width 0.3) (layer "F.Cu") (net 7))
 (segment (start 138.73 100.79) (end 138.73 102.88) (width 0.3) (layer "F.Cu") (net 7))
 (segment (start 111.94 104.05) (end 114.42 106.53) (width 0.3) (layer "F.Cu") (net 7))
 (segment (start 116.82 97.16) (end 114.92 97.16) (width 0.3) (layer "F.Cu") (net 7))
 (segment (start 111.94 99.22) (end 111.94 104.05) (width 0.3) (layer "F.Cu") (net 7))
 (segment (start 124.17 103.71) (end 124.17 103.56) (width 0.3) (layer "F.Cu") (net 7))
 (segment (start 124 103.88) (end 124.32 103.56) (width 0.3) (layer "F.Cu") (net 7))
 (segment (start 123.45 100.75) (end 123.68 100.52) (width 0.3) (layer "F.Cu") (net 7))
 (via (at 123.68 100.52) (size 0.6) (drill 0.3) (layers "F.Cu" "B.Cu") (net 7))
 (via (at 124.17 103.56) (size 0.6) (drill 0.3) (layers "F.Cu" "B.Cu") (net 7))
 (segment (start 124.17 101.01) (end 124.17 103.56) (width 0.3) (layer "B.Cu") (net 7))
 (segment (start 123.68 100.52) (end 124.17 101.01) (width 0.3) (layer "B.Cu") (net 7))
 (segment (start 123.01 101.77) (end 126.84 101.77) (width 0.3) (layer "F.Cu") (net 3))
 (segment (start 121.11 105.69) (end 122.46 104.34) (width 0.3) (layer "F.Cu") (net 3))
 (segment (start 122.46 104.34) (end 122.46 102.32) (width 0.3) (layer "F.Cu") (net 3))
 (segment (start 116.265 97.75) (end 115.33 97.75) (width 0.3) (layer "F.Cu") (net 3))
 (segment (start 112.74 103.72) (end 114.71 105.69) (width 0.3) (layer "F.Cu") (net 3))
 (segment (start 115.33 97.75) (end 114.98 98.1) (width 0.3) (layer "F.Cu") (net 3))
 (segment (start 127.64 102.57) (end 137.775 102.57) (width 0.3) (layer "F.Cu") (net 3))
 (segment (start 114.71 105.69) (end 121.11 105.69) (width 0.3) (layer "F.Cu") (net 3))
 (segment (start 114.98 98.1) (end 114.44 98.1) (width 0.3) (layer "F.Cu") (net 3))
 (segment (start 114.44 98.1) (end 112.74 99.8) (width 0.3) (layer "F.Cu") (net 3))
 (segment (start 112.74 99.8) (end 112.74 103.72) (width 0.3) (layer "F.Cu") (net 3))
 (segment (start 122.46 102.32) (end 123.01 101.77) (width 0.3) (layer "F.Cu") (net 3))
 (segment (start 126.84 101.77) (end 127.64 102.57) (width 0.3) (layer "F.Cu") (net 3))
 (segment (start 122.675 99.25) (end 127.65 99.25) (width 0.3) (layer "F.Cu") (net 6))
 (segment (start 127.65 99.25) (end 129.47 101.07) (width 0.3) (layer "F.Cu") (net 6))
 (segment (start 129.47 101.07) (end 137.775 101.07) (width 0.3) (layer "F.Cu") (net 6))
 (segment (start 116.775 104.965) (end 120.77 104.965) (width 0.3) (layer "F.Cu") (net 13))
 (segment (start 116.265 98.75) (end 114.74 98.75) (width 0.3) (layer "F.Cu") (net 13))
 (segment (start 121.82 103.915) (end 121.82 100.55) (width 0.3) (layer "F.Cu") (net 13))
 (segment (start 114.74 98.75) (end 113.82 99.67) (width 0.3) (layer "F.Cu") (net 13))
 (segment (start 113.82 102.01) (end 116.775 104.965) (width 0.3) (layer "F.Cu") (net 13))
 (segment (start 122.12 100.25) (end 122.675 100.25) (width 0.3) (layer "F.Cu") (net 13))
 (segment (start 121.82 100.55) (end 122.12 100.25) (width 0.3) (layer "F.Cu") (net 13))
 (segment (start 113.82 99.67) (end 113.82 102.01) (width 0.3) (layer "F.Cu") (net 13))
 (segment (start 120.77 104.965) (end 121.82 103.915) (width 0.3) (layer "F.Cu") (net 13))
 (segment (start 128.26 102.07) (end 137.775 102.07) (width 0.3) (layer "F.Cu") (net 4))
 (segment (start 122.675 101.25) (end 127.44 101.25) (width 0.3) (layer "F.Cu") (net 4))
 (segment (start 127.44 101.25) (end 128.26 102.07) (width 0.3) (layer "F.Cu") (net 4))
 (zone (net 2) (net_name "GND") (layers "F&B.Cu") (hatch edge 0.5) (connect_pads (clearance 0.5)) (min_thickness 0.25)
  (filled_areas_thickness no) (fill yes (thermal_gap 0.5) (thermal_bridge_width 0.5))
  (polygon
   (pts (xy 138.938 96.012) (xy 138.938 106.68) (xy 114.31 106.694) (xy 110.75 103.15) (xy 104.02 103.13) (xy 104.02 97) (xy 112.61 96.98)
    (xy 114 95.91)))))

